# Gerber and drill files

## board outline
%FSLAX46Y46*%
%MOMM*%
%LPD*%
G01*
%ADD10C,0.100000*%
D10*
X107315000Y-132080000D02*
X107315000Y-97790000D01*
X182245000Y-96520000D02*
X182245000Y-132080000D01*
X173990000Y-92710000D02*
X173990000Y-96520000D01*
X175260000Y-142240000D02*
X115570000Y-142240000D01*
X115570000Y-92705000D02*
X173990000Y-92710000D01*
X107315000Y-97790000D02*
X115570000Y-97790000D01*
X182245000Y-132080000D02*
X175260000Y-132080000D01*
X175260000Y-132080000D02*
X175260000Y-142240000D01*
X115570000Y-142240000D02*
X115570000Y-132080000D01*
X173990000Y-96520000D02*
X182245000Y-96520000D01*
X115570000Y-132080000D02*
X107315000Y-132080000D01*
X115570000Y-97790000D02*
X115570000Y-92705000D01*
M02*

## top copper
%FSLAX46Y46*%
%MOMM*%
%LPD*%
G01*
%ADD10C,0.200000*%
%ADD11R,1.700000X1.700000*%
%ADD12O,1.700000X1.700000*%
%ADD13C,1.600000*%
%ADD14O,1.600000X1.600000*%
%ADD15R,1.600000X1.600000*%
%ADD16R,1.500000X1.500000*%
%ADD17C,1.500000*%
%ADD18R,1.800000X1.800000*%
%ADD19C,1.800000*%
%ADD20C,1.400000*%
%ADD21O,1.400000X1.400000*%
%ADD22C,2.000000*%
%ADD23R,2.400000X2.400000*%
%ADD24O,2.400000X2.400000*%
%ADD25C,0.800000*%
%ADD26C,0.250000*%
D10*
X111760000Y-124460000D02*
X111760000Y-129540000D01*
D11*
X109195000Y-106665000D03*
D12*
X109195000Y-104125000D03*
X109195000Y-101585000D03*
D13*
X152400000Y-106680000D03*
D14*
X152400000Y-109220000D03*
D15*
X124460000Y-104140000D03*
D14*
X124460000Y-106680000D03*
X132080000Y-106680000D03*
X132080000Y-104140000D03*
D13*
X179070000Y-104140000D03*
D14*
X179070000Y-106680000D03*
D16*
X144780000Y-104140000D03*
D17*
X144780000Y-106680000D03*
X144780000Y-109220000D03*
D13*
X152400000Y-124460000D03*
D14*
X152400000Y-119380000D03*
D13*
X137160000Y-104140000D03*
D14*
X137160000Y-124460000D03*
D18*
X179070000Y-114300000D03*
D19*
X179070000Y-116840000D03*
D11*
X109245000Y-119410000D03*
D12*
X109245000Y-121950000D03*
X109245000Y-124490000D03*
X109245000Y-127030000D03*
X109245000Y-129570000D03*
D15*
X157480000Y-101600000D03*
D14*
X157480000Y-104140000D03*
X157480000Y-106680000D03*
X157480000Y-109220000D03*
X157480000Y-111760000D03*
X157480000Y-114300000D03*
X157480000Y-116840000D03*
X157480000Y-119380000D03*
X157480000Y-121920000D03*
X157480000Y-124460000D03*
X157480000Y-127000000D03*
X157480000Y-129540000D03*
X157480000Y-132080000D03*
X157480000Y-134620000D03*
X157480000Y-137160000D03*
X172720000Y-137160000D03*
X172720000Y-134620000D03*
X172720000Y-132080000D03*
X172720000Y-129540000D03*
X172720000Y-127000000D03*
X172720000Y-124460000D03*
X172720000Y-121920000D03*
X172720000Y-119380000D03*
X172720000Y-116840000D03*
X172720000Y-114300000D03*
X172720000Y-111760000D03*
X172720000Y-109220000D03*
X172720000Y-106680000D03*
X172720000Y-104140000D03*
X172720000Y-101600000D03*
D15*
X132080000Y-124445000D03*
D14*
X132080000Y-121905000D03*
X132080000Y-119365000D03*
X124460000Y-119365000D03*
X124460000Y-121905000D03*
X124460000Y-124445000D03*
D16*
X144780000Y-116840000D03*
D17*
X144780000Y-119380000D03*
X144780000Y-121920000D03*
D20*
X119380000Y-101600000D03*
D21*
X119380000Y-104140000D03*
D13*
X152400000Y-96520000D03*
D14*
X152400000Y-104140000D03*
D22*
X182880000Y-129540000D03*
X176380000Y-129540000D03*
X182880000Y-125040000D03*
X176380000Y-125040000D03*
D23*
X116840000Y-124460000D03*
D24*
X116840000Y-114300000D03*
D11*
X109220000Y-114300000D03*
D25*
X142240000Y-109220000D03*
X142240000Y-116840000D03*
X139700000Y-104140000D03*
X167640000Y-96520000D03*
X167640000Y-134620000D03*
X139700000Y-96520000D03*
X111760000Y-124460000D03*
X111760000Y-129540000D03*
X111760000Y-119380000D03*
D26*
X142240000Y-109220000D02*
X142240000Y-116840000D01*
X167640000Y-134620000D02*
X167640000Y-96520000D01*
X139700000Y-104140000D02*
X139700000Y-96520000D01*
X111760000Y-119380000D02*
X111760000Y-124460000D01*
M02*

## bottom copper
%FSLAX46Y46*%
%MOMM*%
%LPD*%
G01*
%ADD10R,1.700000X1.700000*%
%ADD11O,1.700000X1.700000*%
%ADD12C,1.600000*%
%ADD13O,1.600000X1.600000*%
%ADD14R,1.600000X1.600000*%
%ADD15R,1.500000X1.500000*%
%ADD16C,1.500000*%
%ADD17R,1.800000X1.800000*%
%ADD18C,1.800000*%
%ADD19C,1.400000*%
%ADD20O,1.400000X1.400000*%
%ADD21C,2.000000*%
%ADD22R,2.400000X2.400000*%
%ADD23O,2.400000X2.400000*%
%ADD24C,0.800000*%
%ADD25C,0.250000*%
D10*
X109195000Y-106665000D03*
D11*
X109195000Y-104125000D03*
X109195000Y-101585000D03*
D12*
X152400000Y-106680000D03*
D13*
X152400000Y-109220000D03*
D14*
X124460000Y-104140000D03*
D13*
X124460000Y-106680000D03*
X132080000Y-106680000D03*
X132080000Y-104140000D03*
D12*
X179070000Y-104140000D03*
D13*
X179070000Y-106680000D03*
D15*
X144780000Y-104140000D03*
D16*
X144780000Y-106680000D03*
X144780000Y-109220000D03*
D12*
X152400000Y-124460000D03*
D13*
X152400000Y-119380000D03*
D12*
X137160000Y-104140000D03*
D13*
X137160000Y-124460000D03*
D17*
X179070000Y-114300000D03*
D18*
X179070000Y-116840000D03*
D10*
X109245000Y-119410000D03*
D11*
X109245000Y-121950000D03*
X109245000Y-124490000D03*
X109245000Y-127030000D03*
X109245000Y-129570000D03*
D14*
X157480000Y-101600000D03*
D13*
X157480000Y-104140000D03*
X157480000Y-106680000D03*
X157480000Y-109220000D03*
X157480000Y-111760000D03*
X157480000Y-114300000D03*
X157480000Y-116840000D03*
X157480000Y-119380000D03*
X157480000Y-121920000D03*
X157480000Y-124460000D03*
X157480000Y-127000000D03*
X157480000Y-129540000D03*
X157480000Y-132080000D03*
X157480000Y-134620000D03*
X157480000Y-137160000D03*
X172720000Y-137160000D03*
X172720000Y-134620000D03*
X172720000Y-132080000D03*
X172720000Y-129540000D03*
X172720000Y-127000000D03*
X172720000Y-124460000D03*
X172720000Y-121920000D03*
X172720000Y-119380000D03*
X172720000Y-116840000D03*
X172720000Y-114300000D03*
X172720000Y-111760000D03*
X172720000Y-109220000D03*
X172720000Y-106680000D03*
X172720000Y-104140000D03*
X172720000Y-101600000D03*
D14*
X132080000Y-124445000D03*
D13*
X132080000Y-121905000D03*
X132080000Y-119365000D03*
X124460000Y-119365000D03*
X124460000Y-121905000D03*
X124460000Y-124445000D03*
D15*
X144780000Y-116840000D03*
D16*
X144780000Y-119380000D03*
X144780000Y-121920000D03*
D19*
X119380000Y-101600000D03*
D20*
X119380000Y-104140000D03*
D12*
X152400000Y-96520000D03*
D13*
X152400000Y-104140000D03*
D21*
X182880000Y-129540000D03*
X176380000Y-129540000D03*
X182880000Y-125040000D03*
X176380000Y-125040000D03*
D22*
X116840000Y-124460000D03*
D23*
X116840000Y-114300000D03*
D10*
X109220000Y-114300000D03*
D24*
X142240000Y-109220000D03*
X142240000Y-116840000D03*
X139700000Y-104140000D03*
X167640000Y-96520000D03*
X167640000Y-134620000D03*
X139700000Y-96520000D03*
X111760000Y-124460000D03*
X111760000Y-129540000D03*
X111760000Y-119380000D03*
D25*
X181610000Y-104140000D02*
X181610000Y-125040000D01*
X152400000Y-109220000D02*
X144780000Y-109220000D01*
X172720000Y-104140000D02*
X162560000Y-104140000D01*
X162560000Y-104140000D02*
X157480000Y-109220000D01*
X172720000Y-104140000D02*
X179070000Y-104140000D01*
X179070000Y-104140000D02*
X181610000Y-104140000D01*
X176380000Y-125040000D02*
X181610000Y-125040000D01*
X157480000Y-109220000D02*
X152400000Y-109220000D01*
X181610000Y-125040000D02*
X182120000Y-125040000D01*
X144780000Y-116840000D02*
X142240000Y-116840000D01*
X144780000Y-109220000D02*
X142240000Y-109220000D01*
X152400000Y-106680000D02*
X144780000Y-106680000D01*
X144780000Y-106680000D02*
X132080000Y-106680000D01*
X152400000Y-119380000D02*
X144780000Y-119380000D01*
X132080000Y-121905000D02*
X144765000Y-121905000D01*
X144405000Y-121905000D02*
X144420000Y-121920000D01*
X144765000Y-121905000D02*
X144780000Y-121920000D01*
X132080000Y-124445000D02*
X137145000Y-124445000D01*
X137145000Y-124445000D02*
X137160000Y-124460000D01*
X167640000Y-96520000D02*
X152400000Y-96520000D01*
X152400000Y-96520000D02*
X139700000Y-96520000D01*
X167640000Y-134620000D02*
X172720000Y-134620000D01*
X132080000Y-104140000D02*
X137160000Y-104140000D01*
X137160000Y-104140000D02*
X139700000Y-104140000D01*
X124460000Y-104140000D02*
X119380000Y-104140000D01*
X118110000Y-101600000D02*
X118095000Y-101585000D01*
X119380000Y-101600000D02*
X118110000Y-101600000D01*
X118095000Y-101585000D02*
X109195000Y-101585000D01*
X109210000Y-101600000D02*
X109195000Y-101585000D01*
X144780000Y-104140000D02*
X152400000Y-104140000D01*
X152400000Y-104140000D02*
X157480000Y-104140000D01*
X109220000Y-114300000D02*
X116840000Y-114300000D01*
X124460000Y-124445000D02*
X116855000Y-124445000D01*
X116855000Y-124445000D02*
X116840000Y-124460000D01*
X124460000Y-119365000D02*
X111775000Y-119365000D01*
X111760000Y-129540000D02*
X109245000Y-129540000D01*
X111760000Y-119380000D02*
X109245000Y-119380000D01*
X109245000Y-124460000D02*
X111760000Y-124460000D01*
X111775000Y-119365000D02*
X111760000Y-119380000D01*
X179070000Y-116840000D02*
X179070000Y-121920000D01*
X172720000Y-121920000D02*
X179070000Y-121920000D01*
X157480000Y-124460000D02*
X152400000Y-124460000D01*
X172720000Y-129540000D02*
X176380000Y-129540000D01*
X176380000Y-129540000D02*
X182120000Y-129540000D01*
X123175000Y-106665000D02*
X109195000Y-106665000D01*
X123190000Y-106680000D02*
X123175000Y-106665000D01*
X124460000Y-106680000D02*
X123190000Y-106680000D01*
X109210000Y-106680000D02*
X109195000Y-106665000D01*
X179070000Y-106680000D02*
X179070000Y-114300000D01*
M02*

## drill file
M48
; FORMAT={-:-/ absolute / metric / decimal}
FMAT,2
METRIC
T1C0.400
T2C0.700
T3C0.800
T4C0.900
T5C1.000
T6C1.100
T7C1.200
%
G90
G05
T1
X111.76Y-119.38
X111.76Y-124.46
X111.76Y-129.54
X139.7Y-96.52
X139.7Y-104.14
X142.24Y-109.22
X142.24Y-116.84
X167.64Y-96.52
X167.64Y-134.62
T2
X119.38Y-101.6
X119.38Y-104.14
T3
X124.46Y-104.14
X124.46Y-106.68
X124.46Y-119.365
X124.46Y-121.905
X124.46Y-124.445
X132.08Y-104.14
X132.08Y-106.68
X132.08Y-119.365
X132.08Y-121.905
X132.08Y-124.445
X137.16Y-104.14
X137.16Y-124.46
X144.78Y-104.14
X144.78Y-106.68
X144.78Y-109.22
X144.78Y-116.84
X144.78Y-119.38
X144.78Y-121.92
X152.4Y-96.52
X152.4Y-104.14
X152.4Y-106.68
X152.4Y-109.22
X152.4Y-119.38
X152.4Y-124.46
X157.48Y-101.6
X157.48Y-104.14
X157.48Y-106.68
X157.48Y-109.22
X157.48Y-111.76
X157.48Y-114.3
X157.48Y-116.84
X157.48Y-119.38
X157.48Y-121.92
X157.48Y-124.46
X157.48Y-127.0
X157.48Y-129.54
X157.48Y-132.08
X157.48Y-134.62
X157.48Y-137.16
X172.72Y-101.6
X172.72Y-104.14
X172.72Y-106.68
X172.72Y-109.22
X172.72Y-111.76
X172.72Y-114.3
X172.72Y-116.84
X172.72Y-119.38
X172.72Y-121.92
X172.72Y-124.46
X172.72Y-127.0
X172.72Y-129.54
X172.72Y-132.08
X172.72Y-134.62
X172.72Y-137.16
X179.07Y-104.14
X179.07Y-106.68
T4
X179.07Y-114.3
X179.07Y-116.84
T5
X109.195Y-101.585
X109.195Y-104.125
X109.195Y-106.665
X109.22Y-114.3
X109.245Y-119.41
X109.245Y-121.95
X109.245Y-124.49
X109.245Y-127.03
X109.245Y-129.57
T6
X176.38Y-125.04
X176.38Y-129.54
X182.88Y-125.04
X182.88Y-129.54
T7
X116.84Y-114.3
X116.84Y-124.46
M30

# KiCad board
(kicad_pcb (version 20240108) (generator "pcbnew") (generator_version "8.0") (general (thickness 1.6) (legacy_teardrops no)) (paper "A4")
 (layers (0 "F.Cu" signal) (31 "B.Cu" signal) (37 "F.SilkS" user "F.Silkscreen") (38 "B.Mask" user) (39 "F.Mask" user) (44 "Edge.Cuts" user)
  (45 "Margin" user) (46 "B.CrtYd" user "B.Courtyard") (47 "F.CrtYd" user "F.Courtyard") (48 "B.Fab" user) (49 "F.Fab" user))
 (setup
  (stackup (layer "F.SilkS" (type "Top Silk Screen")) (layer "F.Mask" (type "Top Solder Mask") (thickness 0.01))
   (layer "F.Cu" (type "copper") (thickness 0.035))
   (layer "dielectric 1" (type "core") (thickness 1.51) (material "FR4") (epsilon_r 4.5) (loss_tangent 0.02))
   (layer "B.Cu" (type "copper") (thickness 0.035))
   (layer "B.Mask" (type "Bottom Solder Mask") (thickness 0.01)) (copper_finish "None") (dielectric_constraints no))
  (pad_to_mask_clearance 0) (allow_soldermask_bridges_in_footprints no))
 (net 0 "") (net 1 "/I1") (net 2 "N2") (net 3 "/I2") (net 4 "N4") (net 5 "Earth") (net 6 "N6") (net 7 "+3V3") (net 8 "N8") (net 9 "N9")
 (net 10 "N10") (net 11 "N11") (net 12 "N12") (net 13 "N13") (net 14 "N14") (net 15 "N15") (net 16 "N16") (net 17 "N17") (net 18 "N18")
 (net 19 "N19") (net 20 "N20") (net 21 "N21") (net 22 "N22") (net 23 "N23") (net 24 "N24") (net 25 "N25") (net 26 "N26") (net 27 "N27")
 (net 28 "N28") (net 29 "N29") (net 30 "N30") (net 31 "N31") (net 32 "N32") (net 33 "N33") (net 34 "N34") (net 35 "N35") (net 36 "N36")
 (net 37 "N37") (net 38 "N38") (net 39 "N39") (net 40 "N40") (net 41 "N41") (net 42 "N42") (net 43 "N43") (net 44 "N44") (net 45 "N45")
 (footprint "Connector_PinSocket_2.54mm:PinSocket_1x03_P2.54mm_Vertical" (layer "F.Cu") (at 109.195 106.665 180)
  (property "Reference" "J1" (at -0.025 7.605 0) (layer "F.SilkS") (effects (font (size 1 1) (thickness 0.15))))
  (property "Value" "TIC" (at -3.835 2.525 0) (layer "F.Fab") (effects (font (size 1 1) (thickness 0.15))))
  (pad "1" thru_hole rect (at 0 0 180) (size 1.7 1.7) (drill 1) (layers "*.Cu" "*.Mask") (remove_unused_layers no) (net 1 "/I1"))
  (pad "2" thru_hole oval (at 0 2.54 180) (size 1.7 1.7) (drill 1) (layers "*.Cu" "*.Mask") (remove_unused_layers no) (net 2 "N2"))
  (pad "3" thru_hole oval (at 0 5.08 180) (size 1.7 1.7) (drill 1) (layers "*.Cu" "*.Mask") (remove_unused_layers no) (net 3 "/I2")))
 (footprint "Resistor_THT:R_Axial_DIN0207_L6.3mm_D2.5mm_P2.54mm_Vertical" (layer "F.Cu") (at 152.4 106.68 -90)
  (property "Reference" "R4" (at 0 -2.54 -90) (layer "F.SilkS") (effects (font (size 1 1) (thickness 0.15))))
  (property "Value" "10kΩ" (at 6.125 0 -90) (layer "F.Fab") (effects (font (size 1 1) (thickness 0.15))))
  (pad "1" thru_hole circle (at 0 0 270) (size 1.6 1.6) (drill 0.8) (layers "*.Cu" "*.Mask") (remove_unused_layers no) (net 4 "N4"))
  (pad "2" thru_hole oval (at 2.54 0 270) (size 1.6 1.6) (drill 0.8) (layers "*.Cu" "*.Mask") (remove_unused_layers no) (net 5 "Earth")))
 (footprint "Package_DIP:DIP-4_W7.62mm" (layer "F.Cu") (at 124.46 104.14)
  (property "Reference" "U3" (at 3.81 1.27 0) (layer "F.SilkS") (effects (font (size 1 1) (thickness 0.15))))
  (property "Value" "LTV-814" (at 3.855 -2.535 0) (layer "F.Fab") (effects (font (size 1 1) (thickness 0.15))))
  (pad "1" thru_hole rect (at 0 0) (size 1.6 1.6) (drill 0.8) (layers "*.Cu" "*.Mask") (remove_unused_layers no) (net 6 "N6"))
  (pad "2" thru_hole oval (at 0 2.54) (size 1.6 1.6) (drill 0.8) (layers "*.Cu" "*.Mask") (remove_unused_layers no) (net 1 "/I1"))
  (pad "3" thru_hole oval (at 7.62 2.54) (size 1.6 1.6) (drill 0.8) (layers "*.Cu" "*.Mask") (remove_unused_layers no) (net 4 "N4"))
  (pad "4" thru_hole oval (at 7.62 0) (size 1.6 1.6) (drill 0.8) (layers "*.Cu" "*.Mask") (remove_unused_layers no) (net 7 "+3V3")))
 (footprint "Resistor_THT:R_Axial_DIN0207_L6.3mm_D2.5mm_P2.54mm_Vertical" (layer "F.Cu") (at 179.07 104.14 -90)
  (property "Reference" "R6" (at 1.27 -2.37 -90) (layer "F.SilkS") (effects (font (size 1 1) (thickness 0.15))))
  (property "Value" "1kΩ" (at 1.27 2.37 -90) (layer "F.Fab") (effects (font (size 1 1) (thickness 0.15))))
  (pad "1" thru_hole circle (at 0 0 270) (size 1.6 1.6) (drill 0.8) (layers "*.Cu" "*.Mask") (remove_unused_layers no) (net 5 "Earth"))
  (pad "2" thru_hole oval (at 2.54 0 270) (size 1.6 1.6) (drill 0.8) (layers "*.Cu" "*.Mask") (remove_unused_layers no) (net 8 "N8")))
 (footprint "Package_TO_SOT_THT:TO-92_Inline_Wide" (layer "F.Cu") (at 144.78 104.14 -90)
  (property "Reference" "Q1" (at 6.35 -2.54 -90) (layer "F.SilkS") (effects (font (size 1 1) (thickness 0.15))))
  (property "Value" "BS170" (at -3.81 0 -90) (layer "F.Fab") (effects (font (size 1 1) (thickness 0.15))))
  (pad "1" thru_hole rect (at 0 0 270) (size 1.5 1.5) (drill 0.8) (layers "*.Cu" "*.Mask") (remove_unused_layers no) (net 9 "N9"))
  (pad "2" thru_hole circle (at 2.54 0 270) (size 1.5 1.5) (drill 0.8) (layers "*.Cu" "*.Mask") (remove_unused_layers no) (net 4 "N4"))
  (pad "3" thru_hole circle (at 5.08 0 270) (size 1.5 1.5) (drill 0.8) (layers "*.Cu" "*.Mask") (remove_unused_layers no) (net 5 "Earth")))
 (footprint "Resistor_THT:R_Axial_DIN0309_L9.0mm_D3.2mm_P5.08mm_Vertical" (layer "F.Cu") (at 152.4 124.46 90)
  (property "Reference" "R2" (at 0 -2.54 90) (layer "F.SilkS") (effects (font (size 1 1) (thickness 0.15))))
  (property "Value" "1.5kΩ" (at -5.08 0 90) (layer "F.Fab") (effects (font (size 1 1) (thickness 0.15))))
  (pad "1" thru_hole circle (at 0 0 90) (size 1.6 1.6) (drill 0.8) (layers "*.Cu" "*.Mask") (remove_unused_layers no) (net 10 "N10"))
  (pad "2" thru_hole oval (at 5.08 0 90) (size 1.6 1.6) (drill 0.8) (layers "*.Cu" "*.Mask") (remove_unused_layers no) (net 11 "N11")))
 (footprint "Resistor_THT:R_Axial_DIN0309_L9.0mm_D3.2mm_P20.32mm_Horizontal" (layer "F.Cu") (at 137.16 104.14 -90)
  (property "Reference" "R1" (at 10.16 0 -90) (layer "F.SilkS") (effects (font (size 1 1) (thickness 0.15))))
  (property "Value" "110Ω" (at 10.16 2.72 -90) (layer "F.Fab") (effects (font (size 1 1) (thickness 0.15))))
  (pad "1" thru_hole circle (at 0 0 270) (size 1.6 1.6) (drill 0.8) (layers "*.Cu" "*.Mask") (remove_unused_layers no) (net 7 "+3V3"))
  (pad "2" thru_hole oval (at 20.32 0 270) (size 1.6 1.6) (drill 0.8) (layers "*.Cu" "*.Mask") (remove_unused_layers no) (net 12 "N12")))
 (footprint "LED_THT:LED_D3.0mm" (layer "F.Cu") (at 179.07 114.3 -90)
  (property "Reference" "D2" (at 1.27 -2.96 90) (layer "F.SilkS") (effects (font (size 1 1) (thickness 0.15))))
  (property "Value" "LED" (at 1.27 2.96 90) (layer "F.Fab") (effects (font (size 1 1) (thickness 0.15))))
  (pad "1" thru_hole rect (at 0 0 270) (size 1.8 1.8) (drill 0.9) (layers "*.Cu" "*.Mask") (remove_unused_layers no) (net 8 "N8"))
  (pad "2" thru_hole circle (at 2.54 0 270) (size 1.8 1.8) (drill 0.9) (layers "*.Cu" "*.Mask") (remove_unused_layers no) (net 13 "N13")))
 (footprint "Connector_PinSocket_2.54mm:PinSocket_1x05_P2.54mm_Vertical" (layer "F.Cu") (at 109.245 119.41)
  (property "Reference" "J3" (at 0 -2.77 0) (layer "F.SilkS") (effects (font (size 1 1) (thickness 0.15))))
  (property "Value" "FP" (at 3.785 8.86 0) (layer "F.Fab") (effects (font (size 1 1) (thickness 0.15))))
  (pad "1" thru_hole rect (at 0 0) (size 1.7 1.7) (drill 1) (layers "*.Cu" "*.Mask") (remove_unused_layers no) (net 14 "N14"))
  (pad "2" thru_hole oval (at 0 2.54) (size 1.7 1.7) (drill 1) (layers "*.Cu" "*.Mask") (remove_unused_layers no) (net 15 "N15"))
  (pad "3" thru_hole oval (at 0 5.08) (size 1.7 1.7) (drill 1) (layers "*.Cu" "*.Mask") (remove_unused_layers no) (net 14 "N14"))
  (pad "4" thru_hole oval (at 0 7.62) (size 1.7 1.7) (drill 1) (layers "*.Cu" "*.Mask") (remove_unused_layers no) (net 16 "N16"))
  (pad "5" thru_hole oval (at 0 10.16) (size 1.7 1.7) (drill 1) (layers "*.Cu" "*.Mask") (remove_unused_layers no) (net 14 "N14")))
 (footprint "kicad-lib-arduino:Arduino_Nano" (layer "F.Cu") (at 157.48 101.6)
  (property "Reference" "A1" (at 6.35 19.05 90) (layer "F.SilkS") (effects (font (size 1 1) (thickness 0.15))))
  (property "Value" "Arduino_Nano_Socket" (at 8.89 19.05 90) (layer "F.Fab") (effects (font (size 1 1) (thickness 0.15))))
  (pad "1" thru_hole rect (at 0 0) (size 1.6 1.6) (drill 0.8) (layers "*.Cu" "*.Mask") (remove_unused_layers no) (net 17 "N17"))
  (pad "2" thru_hole oval (at 0 2.54) (size 1.6 1.6) (drill 0.8) (layers "*.Cu" "*.Mask") (remove_unused_layers no) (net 9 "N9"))
  (pad "3" thru_hole oval (at 0 5.08) (size 1.6 1.6) (drill 0.8) (layers "*.Cu" "*.Mask") (remove_unused_layers no) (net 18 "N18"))
  (pad "4" thru_hole oval (at 0 7.62) (size 1.6 1.6) (drill 0.8) (layers "*.Cu" "*.Mask") (remove_unused_layers no) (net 5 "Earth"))
  (pad "5" thru_hole oval (at 0 10.16) (size 1.6 1.6) (drill 0.8) (layers "*.Cu" "*.Mask") (remove_unused_layers no) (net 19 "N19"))
  (pad "6" thru_hole oval (at 0 12.7) (size 1.6 1.6) (drill 0.8) (layers "*.Cu" "*.Mask") (remove_unused_layers no) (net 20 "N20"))
  (pad "7" thru_hole oval (at 0 15.24) (size 1.6 1.6) (drill 0.8) (layers "*.Cu" "*.Mask") (remove_unused_layers no) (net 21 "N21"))
  (pad "8" thru_hole oval (at 0 17.78) (size 1.6 1.6) (drill 0.8) (layers "*.Cu" "*.Mask") (remove_unused_layers no) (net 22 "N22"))
  (pad "9" thru_hole oval (at 0 20.32) (size 1.6 1.6) (drill 0.8) (layers "*.Cu" "*.Mask") (remove_unused_layers no) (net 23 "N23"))
  (pad "10" thru_hole oval (at 0 22.86) (size 1.6 1.6) (drill 0.8) (layers "*.Cu" "*.Mask") (remove_unused_layers no) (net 10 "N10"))
  (pad "11" thru_hole oval (at 0 25.4) (size 1.6 1.6) (drill 0.8) (layers "*.Cu" "*.Mask") (remove_unused_layers no) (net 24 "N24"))
  (pad "12" thru_hole oval (at 0 27.94) (size 1.6 1.6) (drill 0.8) (layers "*.Cu" "*.Mask") (remove_unused_layers no) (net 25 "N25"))
  (pad "13" thru_hole oval (at 0 30.48) (size 1.6 1.6) (drill 0.8) (layers "*.Cu" "*.Mask") (remove_unused_layers no) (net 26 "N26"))
  (pad "14" thru_hole oval (at 0 33.02) (size 1.6 1.6) (drill 0.8) (layers "*.Cu" "*.Mask") (remove_unused_layers no) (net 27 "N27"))
  (pad "15" thru_hole oval (at 0 35.56) (size 1.6 1.6) (drill 0.8) (layers "*.Cu" "*.Mask") (remove_unused_layers no) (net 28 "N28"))
  (pad "16" thru_hole oval (at 15.24 35.56) (size 1.6 1.6) (drill 0.8) (layers "*.Cu" "*.Mask") (remove_unused_layers no) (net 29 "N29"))
  (pad "17" thru_hole oval (at 15.24 33.02) (size 1.6 1.6) (drill 0.8) (layers "*.Cu" "*.Mask") (remove_unused_layers no) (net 7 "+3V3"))
  (pad "18" thru_hole oval (at 15.24 30.48) (size 1.6 1.6) (drill 0.8) (layers "*.Cu" "*.Mask") (remove_unused_layers no) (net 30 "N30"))
  (pad "19" thru_hole oval (at 15.24 27.94) (size 1.6 1.6) (drill 0.8) (layers "*.Cu" "*.Mask") (remove_unused_layers no) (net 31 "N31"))
  (pad "20" thru_hole oval (at 15.24 25.4) (size 1.6 1.6) (drill 0.8) (layers "*.Cu" "*.Mask") (remove_unused_layers no) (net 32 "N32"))
  (pad "21" thru_hole oval (at 15.24 22.86) (size 1.6 1.6) (drill 0.8) (layers "*.Cu" "*.Mask") (remove_unused_layers no) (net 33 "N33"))
  (pad "22" thru_hole oval (at 15.24 20.32) (size 1.6 1.6) (drill 0.8) (layers "*.Cu" "*.Mask") (remove_unused_layers no) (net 13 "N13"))
  (pad "23" thru_hole oval (at 15.24 17.78) (size 1.6 1.6) (drill 0.8) (layers "*.Cu" "*.Mask") (remove_unused_layers no) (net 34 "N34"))
  (pad "24" thru_hole oval (at 15.24 15.24) (size 1.6 1.6) (drill 0.8) (layers "*.Cu" "*.Mask") (remove_unused_layers no) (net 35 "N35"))
  (pad "25" thru_hole oval (at 15.24 12.7) (size 1.6 1.6) (drill 0.8) (layers "*.Cu" "*.Mask") (remove_unused_layers no) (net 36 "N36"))
  (pad "26" thru_hole oval (at 15.24 10.16) (size 1.6 1.6) (drill 0.8) (layers "*.Cu" "*.Mask") (remove_unused_layers no) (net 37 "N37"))
  (pad "27" thru_hole oval (at 15.24 7.62) (size 1.6 1.6) (drill 0.8) (layers "*.Cu" "*.Mask") (remove_unused_layers no) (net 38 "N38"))
  (pad "28" thru_hole oval (at 15.24 5.08) (size 1.6 1.6) (drill 0.8) (layers "*.Cu" "*.Mask") (remove_unused_layers no) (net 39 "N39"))
  (pad "29" thru_hole oval (at 15.24 2.54) (size 1.6 1.6) (drill 0.8) (layers "*.Cu" "*.Mask") (remove_unused_layers no) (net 5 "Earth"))
  (pad "30" thru_hole oval (at 15.24 0) (size 1.6 1.6) (drill 0.8) (layers "*.Cu" "*.Mask") (remove_unused_layers no) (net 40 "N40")))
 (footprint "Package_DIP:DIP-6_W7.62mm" (layer "F.Cu") (at 132.08 124.445 180)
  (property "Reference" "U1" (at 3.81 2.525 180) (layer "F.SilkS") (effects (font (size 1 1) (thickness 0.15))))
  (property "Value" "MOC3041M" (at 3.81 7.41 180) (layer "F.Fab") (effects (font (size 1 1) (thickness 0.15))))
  (pad "1" thru_hole rect (at 0 0 180) (size 1.6 1.6) (drill 0.8) (layers "*.Cu" "*.Mask") (remove_unused_layers no) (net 12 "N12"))
  (pad "2" thru_hole oval (at 0 2.54 180) (size 1.6 1.6) (drill 0.8) (layers "*.Cu" "*.Mask") (remove_unused_layers no) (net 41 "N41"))
  (pad "3" thru_hole oval (at 0 5.08 180) (size 1.6 1.6) (drill 0.8) (layers "*.Cu" "*.Mask") (remove_unused_layers no) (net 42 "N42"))
  (pad "4" thru_hole oval (at 7.62 5.08 180) (size 1.6 1.6) (drill 0.8) (layers "*.Cu" "*.Mask") (remove_unused_layers no) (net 14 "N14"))
  (pad "5" thru_hole oval (at 7.62 2.54 180) (size 1.6 1.6) (drill 0.8) (layers "*.Cu" "*.Mask") (remove_unused_layers no) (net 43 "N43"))
  (pad "6" thru_hole oval (at 7.62 0 180) (size 1.6 1.6) (drill 0.8) (layers "*.Cu" "*.Mask") (remove_unused_layers no) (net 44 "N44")))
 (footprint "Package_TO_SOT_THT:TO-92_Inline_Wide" (layer "F.Cu") (at 144.78 116.84 -90)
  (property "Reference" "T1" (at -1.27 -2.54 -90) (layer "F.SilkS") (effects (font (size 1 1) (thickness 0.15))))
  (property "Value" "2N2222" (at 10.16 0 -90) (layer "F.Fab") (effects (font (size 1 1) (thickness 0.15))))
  (pad "1" thru_hole rect (at 0 0 270) (size 1.5 1.5) (drill 0.8) (layers "*.Cu" "*.Mask") (remove_unused_layers no) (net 5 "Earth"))
  (pad "2" thru_hole circle (at 2.54 0 270) (size 1.5 1.5) (drill 0.8) (layers "*.Cu" "*.Mask") (remove_unused_layers no) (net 11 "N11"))
  (pad "3" thru_hole circle (at 5.08 0 270) (size 1.5 1.5) (drill 0.8) (layers "*.Cu" "*.Mask") (remove_unused_layers no) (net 41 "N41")))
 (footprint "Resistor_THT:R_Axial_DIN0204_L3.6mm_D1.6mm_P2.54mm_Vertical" (layer "F.Cu") (at 119.38 101.6 -90)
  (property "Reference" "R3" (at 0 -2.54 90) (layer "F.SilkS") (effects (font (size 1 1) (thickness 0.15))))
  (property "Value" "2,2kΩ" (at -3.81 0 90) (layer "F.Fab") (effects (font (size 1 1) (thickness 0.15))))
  (pad "1" thru_hole circle (at 0 0 270) (size 1.4 1.4) (drill 0.7) (layers "*.Cu" "*.Mask") (remove_unused_layers no) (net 3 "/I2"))
  (pad "2" thru_hole oval (at 2.54 0 270) (size 1.4 1.4) (drill 0.7) (layers "*.Cu" "*.Mask") (remove_unused_layers no) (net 6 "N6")))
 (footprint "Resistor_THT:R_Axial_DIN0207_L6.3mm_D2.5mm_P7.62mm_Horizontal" (layer "F.Cu") (at 152.4 96.52 -90)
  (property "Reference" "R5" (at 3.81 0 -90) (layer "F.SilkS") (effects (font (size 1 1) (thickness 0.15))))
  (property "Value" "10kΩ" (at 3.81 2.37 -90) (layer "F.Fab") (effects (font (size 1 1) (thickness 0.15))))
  (pad "1" thru_hole circle (at 0 0 270) (size 1.6 1.6) (drill 0.8) (layers "*.Cu" "*.Mask") (remove_unused_layers no) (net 7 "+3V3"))
  (pad "2" thru_hole oval (at 7.62 0 270) (size 1.6 1.6) (drill 0.8) (layers "*.Cu" "*.Mask") (remove_unused_layers no) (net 9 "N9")))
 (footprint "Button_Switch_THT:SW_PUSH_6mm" (layer "F.Cu") (at 182.88 129.54 180)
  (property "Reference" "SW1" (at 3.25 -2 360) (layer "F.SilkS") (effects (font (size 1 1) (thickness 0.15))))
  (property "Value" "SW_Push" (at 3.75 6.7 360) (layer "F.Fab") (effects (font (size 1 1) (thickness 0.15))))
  (pad "1" thru_hole circle (at 0 0 270) (size 2 2) (drill 1.1) (layers "*.Cu" "*.Mask") (remove_unused_layers no) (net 31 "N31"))
  (pad "1" thru_hole circle (at 6.5 0 270) (size 2 2) (drill 1.1) (layers "*.Cu" "*.Mask") (remove_unused_layers no) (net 31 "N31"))
  (pad "2" thru_hole circle (at 0 4.5 270) (size 2 2) (drill 1.1) (layers "*.Cu" "*.Mask") (remove_unused_layers no) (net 5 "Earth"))
  (pad "2" thru_hole circle (at 6.5 4.5 270) (size 2 2) (drill 1.1) (layers "*.Cu" "*.Mask") (remove_unused_layers no) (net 5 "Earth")))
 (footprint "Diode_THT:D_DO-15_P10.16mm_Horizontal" (layer "F.Cu") (at 116.84 124.46 90)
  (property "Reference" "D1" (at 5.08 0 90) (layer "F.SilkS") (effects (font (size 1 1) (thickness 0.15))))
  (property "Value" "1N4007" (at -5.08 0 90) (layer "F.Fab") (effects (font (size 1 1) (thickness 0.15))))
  (pad "1" thru_hole rect (at 0 0 90) (size 2.4 2.4) (drill 1.2) (layers "*.Cu" "*.Mask") (remove_unused_layers no) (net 44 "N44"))
  (pad "2" thru_hole oval (at 10.16 0 90) (size 2.4 2.4) (drill 1.2) (layers "*.Cu" "*.Mask") (remove_unused_layers no) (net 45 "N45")))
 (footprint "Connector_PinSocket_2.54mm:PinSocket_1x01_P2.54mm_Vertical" (layer "F.Cu") (at 109.22 114.3)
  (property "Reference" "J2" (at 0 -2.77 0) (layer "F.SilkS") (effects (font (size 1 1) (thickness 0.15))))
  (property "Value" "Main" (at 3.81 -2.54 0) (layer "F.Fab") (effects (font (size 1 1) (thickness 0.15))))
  (pad "1" thru_hole rect (at 0 0) (size 1.7 1.7) (drill 1) (layers "*.Cu" "*.Mask") (remove_unused_layers no) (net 45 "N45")))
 (gr_line (start 111.76 124.46) (end 111.76 129.54) (stroke (width 0.2) (type default)) (layer "F.Cu") (net 14))
 (gr_line (start 107.315 132.08) (end 107.315 97.79) (stroke (width 0.1) (type default)) (layer "Edge.Cuts"))
 (gr_line (start 182.245 96.52) (end 182.245 132.08) (stroke (width 0.1) (type default)) (layer "Edge.Cuts"))
 (gr_line (start 173.99 92.71) (end 173.99 96.52) (stroke (width 0.1) (type default)) (layer "Edge.Cuts"))
 (gr_line (start 175.26 142.24) (end 115.57 142.24) (stroke (width 0.1) (type default)) (layer "Edge.Cuts"))
 (gr_line (start 115.57 92.705) (end 173.99 92.71) (stroke (width 0.1) (type default)) (layer "Edge.Cuts"))
 (gr_line (start 107.315 97.79) (end 115.57 97.79) (stroke (width 0.1) (type default)) (layer "Edge.Cuts"))
 (gr_line (start 182.245 132.08) (end 175.26 132.08) (stroke (width 0.1) (type default)) (layer "Edge.Cuts"))
 (gr_line (start 175.26 132.08) (end 175.26 142.24) (stroke (width 0.1) (type default)) (layer "Edge.Cuts"))
 (gr_line (start 115.57 142.24) (end 115.57 132.08) (stroke (width 0.1) (type default)) (layer "Edge.Cuts"))
 (gr_line (start 173.99 96.52) (end 182.245 96.52) (stroke (width 0.1) (type default)) (layer "Edge.Cuts"))
 (gr_line (start 115.57 132.08) (end 107.315 132.08) (stroke (width 0.1) (type default)) (layer "Edge.Cuts"))
 (gr_line (start 115.57 97.79) (end 115.57 92.705) (stroke (width 0.1) (type default)) (layer "Edge.Cuts"))
 (segment (start 142.24 109.22) (end 142.24 116.84) (width 0.25) (layer "F.Cu") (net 5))
 (via (at 142.24 109.22) (size 0.8) (drill 0.4) (layers "F.Cu" "B.Cu") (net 5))
 (via (at 142.24 116.84) (size 0.8) (drill 0.4) (layers "F.Cu" "B.Cu") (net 5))
 (segment (start 181.61 104.14) (end 181.61 125.04) (width 0.25) (layer "B.Cu") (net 5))
 (segment (start 152.4 109.22) (end 144.78 109.22) (width 0.25) (layer "B.Cu") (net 5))
 (segment (start 172.72 104.14) (end 162.56 104.14) (width 0.25) (layer "B.Cu") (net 5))
 (segment (start 162.56 104.14) (end 157.48 109.22) (width 0.25) (layer "B.Cu") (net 5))
 (segment (start 172.72 104.14) (end 179.07 104.14) (width 0.25) (layer "B.Cu") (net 5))
 (segment (start 179.07 104.14) (end 181.61 104.14) (width 0.25) (layer "B.Cu") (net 5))
 (segment (start 176.38 125.04) (end 181.61 125.04) (width 0.25) (layer "B.Cu") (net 5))
 (segment (start 157.48 109.22) (end 152.4 109.22) (width 0.25) (layer "B.Cu") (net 5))
 (segment (start 181.61 125.04) (end 182.12 125.04) (width 0.25) (layer "B.Cu") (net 5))
 (segment (start 144.78 116.84) (end 142.24 116.84) (width 0.25) (layer "B.Cu") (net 5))
 (segment (start 144.78 109.22) (end 142.24 109.22) (width 0.25) (layer "B.Cu") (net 5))
 (segment (start 152.4 106.68) (end 144.78 106.68) (width 0.25) (layer "B.Cu") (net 4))
 (segment (start 144.78 106.68) (end 132.08 106.68) (width 0.25) (layer "B.Cu") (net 4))
 (segment (start 152.4 119.38) (end 144.78 119.38) (width 0.25) (layer "B.Cu") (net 11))
 (segment (start 132.08 121.905) (end 144.765 121.905) (width 0.25) (layer "B.Cu") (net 41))
 (segment (start 144.405 121.905) (end 144.42 121.92) (width 0.25) (layer "B.Cu") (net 41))
 (segment (start 144.765 121.905) (end 144.78 121.92) (width 0.25) (layer "B.Cu") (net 41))
 (segment (start 132.08 124.445) (end 137.145 124.445) (width 0.25) (layer "B.Cu") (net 12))
 (segment (start 137.145 124.445) (end 137.16 124.46) (width 0.25) (layer "B.Cu") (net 12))
 (segment (start 167.64 134.62) (end 167.64 96.52) (width 0.25) (layer "F.Cu") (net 7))
 (segment (start 139.7 104.14) (end 139.7 96.52) (width 0.25) (layer "F.Cu") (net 7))
 (via (at 139.7 104.14) (size 0.8) (drill 0.4) (layers "F.Cu" "B.Cu") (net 7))
 (via (at 167.64 96.52) (size 0.8) (drill 0.4) (layers "F.Cu" "B.Cu") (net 7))
 (via (at 167.64 134.62) (size 0.8) (drill 0.4) (layers "F.Cu" "B.Cu") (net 7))
 (via (at 139.7 96.52) (size 0.8) (drill 0.4) (layers "F.Cu" "B.Cu") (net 7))
 (segment (start 167.64 96.52) (end 152.4 96.52) (width 0.25) (layer "B.Cu") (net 7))
 (segment (start 152.4 96.52) (end 139.7 96.52) (width 0.25) (layer "B.Cu") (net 7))
 (segment (start 167.64 134.62) (end 172.72 134.62) (width 0.25) (layer "B.Cu") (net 7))
 (segment (start 132.08 104.14) (end 137.16 104.14) (width 0.25) (layer "B.Cu") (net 7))
 (segment (start 137.16 104.14) (end 139.7 104.14) (width 0.25) (layer "B.Cu") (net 7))
 (segment (start 124.46 104.14) (end 119.38 104.14) (width 0.25) (layer "B.Cu") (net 6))
 (segment (start 118.11 101.6) (end 118.095 101.585) (width 0.25) (layer "B.Cu") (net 3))
 (segment (start 119.38 101.6) (end 118.11 101.6) (width 0.25) (layer "B.Cu") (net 3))
 (segment (start 118.095 101.585) (end 109.195 101.585) (width 0.25) (layer "B.Cu") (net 3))
 (segment (start 109.21 101.6) (end 109.195 101.585) (width 0.25) (layer "B.Cu") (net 3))
 (segment (start 144.78 104.14) (end 152.4 104.14) (width 0.25) (layer "B.Cu") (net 9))
 (segment (start 152.4 104.14) (end 157.48 104.14) (width 0.25) (layer "B.Cu") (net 9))
 (segment (start 109.22 114.3) (end 116.84 114.3) (width 0.25) (layer "B.Cu") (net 45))
 (segment (start 124.46 124.445) (end 116.855 124.445) (width 0.25) (layer "B.Cu") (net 44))
 (segment (start 116.855 124.445) (end 116.84 124.46) (width 0.25) (layer "B.Cu") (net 44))
 (segment (start 111.76 119.38) (end 111.76 124.46) (width 0.25) (layer "F.Cu") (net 14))
 (via (at 111.76 124.46) (size 0.8) (drill 0.4) (layers "F.Cu" "B.Cu") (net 14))
 (via (at 111.76 129.54) (size 0.8) (drill 0.4) (layers "F.Cu" "B.Cu") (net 14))
 (via (at 111.76 119.38) (size 0.8) (drill 0.4) (layers "F.Cu" "B.Cu") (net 14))
 (segment (start 124.46 119.365) (end 111.775 119.365) (width 0.25) (layer "B.Cu") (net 14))
 (segment (start 111.76 129.54) (end 109.245 129.54) (width 0.25) (layer "B.Cu") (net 14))
 (segment (start 111.76 119.38) (end 109.245 119.38) (width 0.25) (layer "B.Cu") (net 14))
 (segment (start 109.245 124.46) (end 111.76 124.46) (width 0.25) (layer "B.Cu") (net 14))
 (segment (start 111.775 119.365) (end 111.76 119.38) (width 0.25) (layer "B.Cu") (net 14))
 (segment (start 179.07 116.84) (end 179.07 121.92) (width 0.25) (layer "B.Cu") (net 13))
 (segment (start 172.72 121.92) (end 179.07 121.92) (width 0.25) (layer "B.Cu") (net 13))
 (segment (start 157.48 124.46) (end 152.4 124.46) (width 0.25) (layer "B.Cu") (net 10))
 (segment (start 172.72 129.54) (end 176.38 129.54) (width 0.25) (layer "B.Cu") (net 31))
 (segment (start 176.38 129.54) (end 182.12 129.54) (width 0.25) (layer "B.Cu") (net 31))
 (segment (start 123.175 106.665) (end 109.195 106.665) (width 0.25) (layer "B.Cu") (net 1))
 (segment (start 123.19 106.68) (end 123.175 106.665) (width 0.25) (layer "B.Cu") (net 1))
 (segment (start 124.46 106.68) (end 123.19 106.68) (width 0.25) (layer "B.Cu") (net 1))
 (segment (start 109.21 106.68) (end 109.195 106.665) (width 0.25) (layer "B.Cu") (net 1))
 (segment (start 179.07 106.68) (end 179.07 114.3) (width 0.25) (layer "B.Cu") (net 8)))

